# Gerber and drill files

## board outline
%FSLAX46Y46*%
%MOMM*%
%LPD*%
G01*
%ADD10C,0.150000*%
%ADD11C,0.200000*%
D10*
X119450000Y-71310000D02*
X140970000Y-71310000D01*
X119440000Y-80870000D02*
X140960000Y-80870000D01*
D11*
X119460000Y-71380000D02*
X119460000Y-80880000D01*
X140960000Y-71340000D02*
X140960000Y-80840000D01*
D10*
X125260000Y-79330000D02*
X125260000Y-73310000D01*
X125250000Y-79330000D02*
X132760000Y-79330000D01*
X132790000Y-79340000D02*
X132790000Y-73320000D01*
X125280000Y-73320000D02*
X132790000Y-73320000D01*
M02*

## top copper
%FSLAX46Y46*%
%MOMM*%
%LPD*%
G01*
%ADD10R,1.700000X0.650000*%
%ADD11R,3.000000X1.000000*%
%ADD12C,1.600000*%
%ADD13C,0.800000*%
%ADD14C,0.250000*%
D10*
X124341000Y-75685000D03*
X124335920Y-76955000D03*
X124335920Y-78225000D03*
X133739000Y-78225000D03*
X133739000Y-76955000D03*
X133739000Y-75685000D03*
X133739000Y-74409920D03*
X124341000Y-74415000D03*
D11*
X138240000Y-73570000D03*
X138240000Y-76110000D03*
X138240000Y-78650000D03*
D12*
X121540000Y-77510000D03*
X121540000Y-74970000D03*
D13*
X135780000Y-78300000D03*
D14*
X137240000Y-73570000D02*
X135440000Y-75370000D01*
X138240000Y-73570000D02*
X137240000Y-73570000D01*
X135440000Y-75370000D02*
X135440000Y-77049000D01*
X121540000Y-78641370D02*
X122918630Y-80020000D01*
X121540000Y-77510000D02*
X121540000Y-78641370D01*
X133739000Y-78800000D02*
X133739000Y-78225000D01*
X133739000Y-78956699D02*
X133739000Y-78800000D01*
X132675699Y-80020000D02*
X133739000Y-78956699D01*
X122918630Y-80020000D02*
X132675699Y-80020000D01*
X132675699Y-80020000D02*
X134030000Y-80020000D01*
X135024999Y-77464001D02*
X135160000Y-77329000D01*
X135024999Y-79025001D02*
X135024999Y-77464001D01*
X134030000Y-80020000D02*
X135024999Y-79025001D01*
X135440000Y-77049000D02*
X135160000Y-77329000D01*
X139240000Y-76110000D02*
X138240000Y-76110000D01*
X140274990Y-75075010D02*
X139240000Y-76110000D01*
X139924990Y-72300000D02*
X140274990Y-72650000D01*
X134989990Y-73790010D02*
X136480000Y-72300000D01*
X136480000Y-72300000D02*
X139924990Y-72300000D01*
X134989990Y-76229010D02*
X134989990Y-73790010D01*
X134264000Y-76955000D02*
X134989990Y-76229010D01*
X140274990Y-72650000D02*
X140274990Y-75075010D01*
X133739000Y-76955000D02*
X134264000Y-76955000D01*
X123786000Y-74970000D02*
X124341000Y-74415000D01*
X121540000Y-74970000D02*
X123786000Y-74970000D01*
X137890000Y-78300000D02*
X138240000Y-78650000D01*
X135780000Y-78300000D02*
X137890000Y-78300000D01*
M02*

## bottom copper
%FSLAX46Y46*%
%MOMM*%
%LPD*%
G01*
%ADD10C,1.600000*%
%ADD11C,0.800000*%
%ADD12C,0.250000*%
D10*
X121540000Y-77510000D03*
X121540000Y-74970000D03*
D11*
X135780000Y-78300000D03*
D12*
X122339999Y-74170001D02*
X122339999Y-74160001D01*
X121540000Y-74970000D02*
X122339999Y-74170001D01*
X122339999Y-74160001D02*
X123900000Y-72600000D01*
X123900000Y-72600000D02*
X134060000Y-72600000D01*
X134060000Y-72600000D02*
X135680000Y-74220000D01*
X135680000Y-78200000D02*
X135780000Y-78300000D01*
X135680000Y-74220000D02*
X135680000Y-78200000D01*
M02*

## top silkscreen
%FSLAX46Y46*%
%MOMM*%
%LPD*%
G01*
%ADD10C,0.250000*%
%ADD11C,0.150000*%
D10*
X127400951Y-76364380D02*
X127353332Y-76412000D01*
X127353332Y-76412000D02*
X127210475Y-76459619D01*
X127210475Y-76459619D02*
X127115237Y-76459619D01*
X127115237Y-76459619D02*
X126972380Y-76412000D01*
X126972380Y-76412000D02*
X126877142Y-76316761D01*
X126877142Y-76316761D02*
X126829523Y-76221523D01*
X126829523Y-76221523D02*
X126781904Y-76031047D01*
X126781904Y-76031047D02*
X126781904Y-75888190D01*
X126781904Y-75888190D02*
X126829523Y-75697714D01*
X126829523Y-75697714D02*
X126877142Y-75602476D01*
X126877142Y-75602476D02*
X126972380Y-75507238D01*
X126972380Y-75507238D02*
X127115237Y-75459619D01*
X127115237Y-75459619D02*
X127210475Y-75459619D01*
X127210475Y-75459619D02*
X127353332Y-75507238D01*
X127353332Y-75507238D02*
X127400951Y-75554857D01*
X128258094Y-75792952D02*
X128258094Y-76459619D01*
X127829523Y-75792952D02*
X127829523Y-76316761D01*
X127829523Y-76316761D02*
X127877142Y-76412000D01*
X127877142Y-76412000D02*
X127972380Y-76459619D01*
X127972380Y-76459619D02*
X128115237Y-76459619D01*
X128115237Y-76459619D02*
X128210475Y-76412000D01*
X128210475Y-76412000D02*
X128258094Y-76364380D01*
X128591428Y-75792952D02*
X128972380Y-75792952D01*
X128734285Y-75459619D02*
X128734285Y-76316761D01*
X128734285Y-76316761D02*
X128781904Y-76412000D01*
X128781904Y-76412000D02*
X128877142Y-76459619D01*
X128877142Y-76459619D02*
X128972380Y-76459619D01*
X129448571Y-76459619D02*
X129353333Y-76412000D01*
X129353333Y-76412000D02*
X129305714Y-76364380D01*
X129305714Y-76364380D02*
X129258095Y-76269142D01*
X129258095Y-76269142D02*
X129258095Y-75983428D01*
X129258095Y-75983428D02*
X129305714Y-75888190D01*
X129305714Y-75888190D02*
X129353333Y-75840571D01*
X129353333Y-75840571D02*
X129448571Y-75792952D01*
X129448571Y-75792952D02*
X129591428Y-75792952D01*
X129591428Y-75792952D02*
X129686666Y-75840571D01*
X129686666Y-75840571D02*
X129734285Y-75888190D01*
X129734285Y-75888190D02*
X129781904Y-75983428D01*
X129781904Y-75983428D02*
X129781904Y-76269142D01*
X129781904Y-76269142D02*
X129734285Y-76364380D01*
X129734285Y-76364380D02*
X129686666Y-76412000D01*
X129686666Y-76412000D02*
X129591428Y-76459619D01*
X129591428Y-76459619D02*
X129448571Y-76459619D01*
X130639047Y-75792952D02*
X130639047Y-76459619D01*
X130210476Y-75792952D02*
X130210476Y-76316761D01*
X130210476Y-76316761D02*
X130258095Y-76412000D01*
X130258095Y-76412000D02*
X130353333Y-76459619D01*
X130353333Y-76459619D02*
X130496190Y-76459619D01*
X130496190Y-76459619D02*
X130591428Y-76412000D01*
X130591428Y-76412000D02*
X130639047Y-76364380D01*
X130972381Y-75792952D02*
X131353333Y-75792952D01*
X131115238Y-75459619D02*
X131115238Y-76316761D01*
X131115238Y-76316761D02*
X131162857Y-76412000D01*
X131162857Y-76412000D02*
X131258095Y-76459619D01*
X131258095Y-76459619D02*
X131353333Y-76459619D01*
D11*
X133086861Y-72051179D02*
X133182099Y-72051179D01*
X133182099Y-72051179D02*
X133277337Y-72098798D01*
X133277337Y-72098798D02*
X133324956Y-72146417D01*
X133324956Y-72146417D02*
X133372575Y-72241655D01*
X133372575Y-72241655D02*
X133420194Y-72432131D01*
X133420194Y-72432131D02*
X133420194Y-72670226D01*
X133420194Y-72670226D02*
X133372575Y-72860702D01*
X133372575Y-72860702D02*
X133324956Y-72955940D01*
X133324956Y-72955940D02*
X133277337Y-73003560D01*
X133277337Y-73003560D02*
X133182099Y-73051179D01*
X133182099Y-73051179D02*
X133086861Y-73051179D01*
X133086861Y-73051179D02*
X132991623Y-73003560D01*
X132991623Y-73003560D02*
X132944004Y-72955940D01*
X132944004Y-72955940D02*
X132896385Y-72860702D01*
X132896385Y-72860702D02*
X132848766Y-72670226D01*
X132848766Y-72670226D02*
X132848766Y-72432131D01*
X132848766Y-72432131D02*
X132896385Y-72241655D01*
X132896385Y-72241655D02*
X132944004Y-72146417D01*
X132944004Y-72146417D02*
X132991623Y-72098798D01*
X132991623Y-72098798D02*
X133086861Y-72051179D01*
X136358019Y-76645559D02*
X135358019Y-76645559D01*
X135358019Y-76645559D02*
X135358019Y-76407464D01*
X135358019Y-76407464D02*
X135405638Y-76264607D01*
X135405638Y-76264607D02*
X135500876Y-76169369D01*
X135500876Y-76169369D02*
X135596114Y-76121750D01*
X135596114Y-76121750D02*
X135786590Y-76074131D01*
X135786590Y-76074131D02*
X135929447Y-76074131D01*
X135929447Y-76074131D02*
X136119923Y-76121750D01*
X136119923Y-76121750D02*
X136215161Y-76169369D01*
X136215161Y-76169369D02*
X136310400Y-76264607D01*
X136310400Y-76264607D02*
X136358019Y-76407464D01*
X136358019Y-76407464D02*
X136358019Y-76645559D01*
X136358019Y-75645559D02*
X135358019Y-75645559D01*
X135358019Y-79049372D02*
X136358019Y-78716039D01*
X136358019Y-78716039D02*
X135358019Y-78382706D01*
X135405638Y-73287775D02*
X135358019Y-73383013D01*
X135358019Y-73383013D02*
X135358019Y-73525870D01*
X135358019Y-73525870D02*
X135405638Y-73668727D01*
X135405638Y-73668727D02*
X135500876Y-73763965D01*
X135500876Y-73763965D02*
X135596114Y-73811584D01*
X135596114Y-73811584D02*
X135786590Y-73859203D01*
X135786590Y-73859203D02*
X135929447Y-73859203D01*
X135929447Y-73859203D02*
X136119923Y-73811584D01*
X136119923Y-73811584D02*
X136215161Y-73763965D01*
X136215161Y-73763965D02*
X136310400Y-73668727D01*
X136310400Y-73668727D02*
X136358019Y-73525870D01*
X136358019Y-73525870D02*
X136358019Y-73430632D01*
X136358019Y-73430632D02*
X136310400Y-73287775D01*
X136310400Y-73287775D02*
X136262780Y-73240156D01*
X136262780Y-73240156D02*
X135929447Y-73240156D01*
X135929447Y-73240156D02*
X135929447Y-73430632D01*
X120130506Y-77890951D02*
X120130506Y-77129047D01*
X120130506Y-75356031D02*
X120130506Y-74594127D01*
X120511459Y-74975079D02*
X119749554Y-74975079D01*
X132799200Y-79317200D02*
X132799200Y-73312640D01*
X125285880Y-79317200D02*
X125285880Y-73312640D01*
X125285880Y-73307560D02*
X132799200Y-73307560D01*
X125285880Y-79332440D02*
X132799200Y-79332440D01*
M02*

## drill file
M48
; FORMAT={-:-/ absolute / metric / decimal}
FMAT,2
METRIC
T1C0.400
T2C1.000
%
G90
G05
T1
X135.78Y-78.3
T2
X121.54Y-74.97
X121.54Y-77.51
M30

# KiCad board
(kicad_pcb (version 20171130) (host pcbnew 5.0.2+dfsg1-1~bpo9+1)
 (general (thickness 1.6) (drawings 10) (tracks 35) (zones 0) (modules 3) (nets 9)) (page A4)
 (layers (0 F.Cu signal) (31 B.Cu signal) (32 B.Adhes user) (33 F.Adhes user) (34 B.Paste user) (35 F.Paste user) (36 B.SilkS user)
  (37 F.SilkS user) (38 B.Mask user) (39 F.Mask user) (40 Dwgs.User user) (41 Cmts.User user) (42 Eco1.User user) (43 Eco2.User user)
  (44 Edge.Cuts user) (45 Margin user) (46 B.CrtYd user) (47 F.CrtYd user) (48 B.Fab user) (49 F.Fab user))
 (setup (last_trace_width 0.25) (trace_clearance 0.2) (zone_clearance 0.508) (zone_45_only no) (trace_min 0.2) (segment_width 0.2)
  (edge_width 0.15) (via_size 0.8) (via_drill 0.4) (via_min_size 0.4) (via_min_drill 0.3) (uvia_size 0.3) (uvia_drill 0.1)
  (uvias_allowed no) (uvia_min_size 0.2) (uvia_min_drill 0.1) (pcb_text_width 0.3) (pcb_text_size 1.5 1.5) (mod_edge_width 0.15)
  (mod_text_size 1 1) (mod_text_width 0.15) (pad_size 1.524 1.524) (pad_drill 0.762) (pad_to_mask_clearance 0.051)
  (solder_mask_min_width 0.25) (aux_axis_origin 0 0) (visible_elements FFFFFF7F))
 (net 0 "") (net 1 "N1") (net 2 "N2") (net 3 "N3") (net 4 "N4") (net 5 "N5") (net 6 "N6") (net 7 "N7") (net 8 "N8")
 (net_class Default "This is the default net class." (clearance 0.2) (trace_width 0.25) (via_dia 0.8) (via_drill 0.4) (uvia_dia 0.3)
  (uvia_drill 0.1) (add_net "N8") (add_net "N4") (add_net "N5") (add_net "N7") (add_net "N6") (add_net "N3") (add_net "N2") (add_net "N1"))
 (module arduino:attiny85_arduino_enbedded (layer F.Cu) (at 129.04 76.32)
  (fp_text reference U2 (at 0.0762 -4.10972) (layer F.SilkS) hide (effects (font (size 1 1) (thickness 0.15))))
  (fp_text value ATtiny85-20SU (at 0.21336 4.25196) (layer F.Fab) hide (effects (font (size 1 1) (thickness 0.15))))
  (fp_line (start 3.7592 2.9972) (end 3.7592 -3.00736) (layer F.SilkS) (width 0.15))
  (fp_line (start -3.75412 2.9972) (end -3.75412 -3.00736) (layer F.SilkS) (width 0.15))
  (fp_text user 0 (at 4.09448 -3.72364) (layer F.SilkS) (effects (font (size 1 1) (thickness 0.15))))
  (fp_line (start -3.75412 -3.01244) (end 3.7592 -3.01244) (layer F.SilkS) (width 0.15))
  (fp_line (start -3.75412 3.01244) (end 3.7592 3.01244) (layer F.SilkS) (width 0.15))
  (pad 7 smd rect (at -4.699 -0.635) (size 1.7 0.65) (layers F.Cu F.Paste F.Mask) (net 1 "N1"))
  (pad 6 smd rect (at -4.70408 0.635) (size 1.7 0.65) (layers F.Cu F.Paste F.Mask) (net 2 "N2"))
  (pad 5 smd rect (at -4.70408 1.905) (size 1.7 0.65) (layers F.Cu F.Paste F.Mask) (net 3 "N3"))
  (pad 4 smd rect (at 4.699 1.905) (size 1.7 0.65) (layers F.Cu F.Paste F.Mask) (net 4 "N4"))
  (pad 3 smd rect (at 4.699 0.635) (size 1.7 0.65) (layers F.Cu F.Paste F.Mask) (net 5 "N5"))
  (pad 2 smd rect (at 4.699 -0.635) (size 1.7 0.65) (layers F.Cu F.Paste F.Mask) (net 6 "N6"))
  (pad 1 smd rect (at 4.699 -1.91008) (size 1.7 0.65) (layers F.Cu F.Paste F.Mask) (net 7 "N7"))
  (pad 8 smd rect (at -4.699 -1.905) (size 1.7 0.65) (layers F.Cu F.Paste F.Mask) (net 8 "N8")))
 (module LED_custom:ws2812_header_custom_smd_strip (layer F.Cu) (at 138.24 76.11 270)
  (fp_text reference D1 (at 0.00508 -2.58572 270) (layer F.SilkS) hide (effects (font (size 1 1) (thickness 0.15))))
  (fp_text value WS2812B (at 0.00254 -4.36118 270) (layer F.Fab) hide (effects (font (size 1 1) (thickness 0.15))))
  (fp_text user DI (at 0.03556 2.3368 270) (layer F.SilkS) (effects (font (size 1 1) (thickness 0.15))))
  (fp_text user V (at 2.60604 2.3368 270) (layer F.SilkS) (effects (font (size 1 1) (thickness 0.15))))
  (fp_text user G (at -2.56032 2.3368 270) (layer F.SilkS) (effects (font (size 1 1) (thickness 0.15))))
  (pad 3 smd rect (at -2.54 0 270) (size 1 3) (layers F.Cu F.Paste F.Mask) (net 4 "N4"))
  (pad 4 smd rect (at 0 0 270) (size 1 3) (layers F.Cu F.Paste F.Mask) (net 5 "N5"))
  (pad 1 smd rect (at 2.54 0 270) (size 1 3) (layers F.Cu F.Paste F.Mask) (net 8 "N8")))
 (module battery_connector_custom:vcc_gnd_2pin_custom (layer F.Cu) (at 121.54 76.24 90)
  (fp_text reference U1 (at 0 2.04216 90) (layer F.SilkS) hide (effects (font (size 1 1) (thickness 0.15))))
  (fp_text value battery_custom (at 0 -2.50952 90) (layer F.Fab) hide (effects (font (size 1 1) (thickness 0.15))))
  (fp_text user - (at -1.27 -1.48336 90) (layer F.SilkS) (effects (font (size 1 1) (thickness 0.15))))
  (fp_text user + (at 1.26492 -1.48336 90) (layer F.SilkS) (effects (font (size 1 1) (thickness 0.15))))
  (pad 1 thru_hole circle (at -1.27 0 90) (size 1.6 1.6) (drill 1) (layers *.Cu *.Mask) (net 4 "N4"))
  (pad 2 thru_hole circle (at 1.27 0 90) (size 1.6 1.6) (drill 1) (layers *.Cu *.Mask) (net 8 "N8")))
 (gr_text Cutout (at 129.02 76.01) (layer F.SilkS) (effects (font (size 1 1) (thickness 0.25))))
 (gr_line (start 119.45 71.31) (end 140.97 71.31) (layer Edge.Cuts) (width 0.15))
 (gr_line (start 119.44 80.87) (end 140.96 80.87) (layer Edge.Cuts) (width 0.15))
 (gr_line (start 119.46 71.38) (end 119.46 80.88) (layer Edge.Cuts) (width 0.2))
 (gr_line (start 140.96 71.34) (end 140.96 80.84) (layer Edge.Cuts) (width 0.2))
 (gr_line (start 125.26 79.33) (end 125.26 73.31) (layer Edge.Cuts) (width 0.15))
 (gr_line (start 125.25 79.33) (end 132.76 79.33) (layer Edge.Cuts) (width 0.15))
 (gr_line (start 132.79 79.34) (end 132.79 73.32) (layer Edge.Cuts) (width 0.15))
 (gr_line (start 125.28 73.32) (end 132.79 73.32) (layer Edge.Cuts) (width 0.15))
 (segment (start 137.24 73.57) (end 135.44 75.37) (width 0.25) (layer F.Cu) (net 4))
 (segment (start 138.24 73.57) (end 137.24 73.57) (width 0.25) (layer F.Cu) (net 4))
 (segment (start 135.44 75.37) (end 135.44 77.049) (width 0.25) (layer F.Cu) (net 4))
 (segment (start 121.54 78.64137) (end 122.91863 80.02) (width 0.25) (layer F.Cu) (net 4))
 (segment (start 121.54 77.51) (end 121.54 78.64137) (width 0.25) (layer F.Cu) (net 4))
 (segment (start 133.739 78.8) (end 133.739 78.225) (width 0.25) (layer F.Cu) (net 4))
 (segment (start 133.739 78.956699) (end 133.739 78.8) (width 0.25) (layer F.Cu) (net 4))
 (segment (start 132.675699 80.02) (end 133.739 78.956699) (width 0.25) (layer F.Cu) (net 4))
 (segment (start 122.91863 80.02) (end 132.675699 80.02) (width 0.25) (layer F.Cu) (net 4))
 (segment (start 132.675699 80.02) (end 134.03 80.02) (width 0.25) (layer F.Cu) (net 4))
 (segment (start 135.024999 77.464001) (end 135.16 77.329) (width 0.25) (layer F.Cu) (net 4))
 (segment (start 135.024999 79.025001) (end 135.024999 77.464001) (width 0.25) (layer F.Cu) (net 4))
 (segment (start 134.03 80.02) (end 135.024999 79.025001) (width 0.25) (layer F.Cu) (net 4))
 (segment (start 135.44 77.049) (end 135.16 77.329) (width 0.25) (layer F.Cu) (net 4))
 (segment (start 139.24 76.11) (end 138.24 76.11) (width 0.25) (layer F.Cu) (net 5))
 (segment (start 140.27499 75.07501) (end 139.24 76.11) (width 0.25) (layer F.Cu) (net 5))
 (segment (start 139.92499 72.3) (end 140.27499 72.65) (width 0.25) (layer F.Cu) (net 5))
 (segment (start 134.98999 73.79001) (end 136.48 72.3) (width 0.25) (layer F.Cu) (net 5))
 (segment (start 136.48 72.3) (end 139.92499 72.3) (width 0.25) (layer F.Cu) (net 5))
 (segment (start 134.98999 76.22901) (end 134.98999 73.79001) (width 0.25) (layer F.Cu) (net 5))
 (segment (start 134.264 76.955) (end 134.98999 76.22901) (width 0.25) (layer F.Cu) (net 5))
 (segment (start 140.27499 72.65) (end 140.27499 75.07501) (width 0.25) (layer F.Cu) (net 5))
 (segment (start 133.739 76.955) (end 134.264 76.955) (width 0.25) (layer F.Cu) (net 5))
 (segment (start 123.786 74.97) (end 124.341 74.415) (width 0.25) (layer F.Cu) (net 8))
 (segment (start 121.54 74.97) (end 123.786 74.97) (width 0.25) (layer F.Cu) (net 8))
 (segment (start 122.339999 74.170001) (end 122.339999 74.160001) (width 0.25) (layer B.Cu) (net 8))
 (segment (start 121.54 74.97) (end 122.339999 74.170001) (width 0.25) (layer B.Cu) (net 8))
 (segment (start 122.339999 74.160001) (end 123.9 72.6) (width 0.25) (layer B.Cu) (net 8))
 (segment (start 123.9 72.6) (end 134.06 72.6) (width 0.25) (layer B.Cu) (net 8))
 (segment (start 134.06 72.6) (end 135.68 74.22) (width 0.25) (layer B.Cu) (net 8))
 (via (at 135.78 78.3) (size 0.8) (drill 0.4) (layers F.Cu B.Cu) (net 8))
 (segment (start 135.68 78.2) (end 135.78 78.3) (width 0.25) (layer B.Cu) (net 8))
 (segment (start 135.68 74.22) (end 135.68 78.2) (width 0.25) (layer B.Cu) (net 8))
 (segment (start 137.89 78.3) (end 138.24 78.65) (width 0.25) (layer F.Cu) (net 8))
 (segment (start 135.78 78.3) (end 137.89 78.3) (width 0.25) (layer F.Cu) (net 8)))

